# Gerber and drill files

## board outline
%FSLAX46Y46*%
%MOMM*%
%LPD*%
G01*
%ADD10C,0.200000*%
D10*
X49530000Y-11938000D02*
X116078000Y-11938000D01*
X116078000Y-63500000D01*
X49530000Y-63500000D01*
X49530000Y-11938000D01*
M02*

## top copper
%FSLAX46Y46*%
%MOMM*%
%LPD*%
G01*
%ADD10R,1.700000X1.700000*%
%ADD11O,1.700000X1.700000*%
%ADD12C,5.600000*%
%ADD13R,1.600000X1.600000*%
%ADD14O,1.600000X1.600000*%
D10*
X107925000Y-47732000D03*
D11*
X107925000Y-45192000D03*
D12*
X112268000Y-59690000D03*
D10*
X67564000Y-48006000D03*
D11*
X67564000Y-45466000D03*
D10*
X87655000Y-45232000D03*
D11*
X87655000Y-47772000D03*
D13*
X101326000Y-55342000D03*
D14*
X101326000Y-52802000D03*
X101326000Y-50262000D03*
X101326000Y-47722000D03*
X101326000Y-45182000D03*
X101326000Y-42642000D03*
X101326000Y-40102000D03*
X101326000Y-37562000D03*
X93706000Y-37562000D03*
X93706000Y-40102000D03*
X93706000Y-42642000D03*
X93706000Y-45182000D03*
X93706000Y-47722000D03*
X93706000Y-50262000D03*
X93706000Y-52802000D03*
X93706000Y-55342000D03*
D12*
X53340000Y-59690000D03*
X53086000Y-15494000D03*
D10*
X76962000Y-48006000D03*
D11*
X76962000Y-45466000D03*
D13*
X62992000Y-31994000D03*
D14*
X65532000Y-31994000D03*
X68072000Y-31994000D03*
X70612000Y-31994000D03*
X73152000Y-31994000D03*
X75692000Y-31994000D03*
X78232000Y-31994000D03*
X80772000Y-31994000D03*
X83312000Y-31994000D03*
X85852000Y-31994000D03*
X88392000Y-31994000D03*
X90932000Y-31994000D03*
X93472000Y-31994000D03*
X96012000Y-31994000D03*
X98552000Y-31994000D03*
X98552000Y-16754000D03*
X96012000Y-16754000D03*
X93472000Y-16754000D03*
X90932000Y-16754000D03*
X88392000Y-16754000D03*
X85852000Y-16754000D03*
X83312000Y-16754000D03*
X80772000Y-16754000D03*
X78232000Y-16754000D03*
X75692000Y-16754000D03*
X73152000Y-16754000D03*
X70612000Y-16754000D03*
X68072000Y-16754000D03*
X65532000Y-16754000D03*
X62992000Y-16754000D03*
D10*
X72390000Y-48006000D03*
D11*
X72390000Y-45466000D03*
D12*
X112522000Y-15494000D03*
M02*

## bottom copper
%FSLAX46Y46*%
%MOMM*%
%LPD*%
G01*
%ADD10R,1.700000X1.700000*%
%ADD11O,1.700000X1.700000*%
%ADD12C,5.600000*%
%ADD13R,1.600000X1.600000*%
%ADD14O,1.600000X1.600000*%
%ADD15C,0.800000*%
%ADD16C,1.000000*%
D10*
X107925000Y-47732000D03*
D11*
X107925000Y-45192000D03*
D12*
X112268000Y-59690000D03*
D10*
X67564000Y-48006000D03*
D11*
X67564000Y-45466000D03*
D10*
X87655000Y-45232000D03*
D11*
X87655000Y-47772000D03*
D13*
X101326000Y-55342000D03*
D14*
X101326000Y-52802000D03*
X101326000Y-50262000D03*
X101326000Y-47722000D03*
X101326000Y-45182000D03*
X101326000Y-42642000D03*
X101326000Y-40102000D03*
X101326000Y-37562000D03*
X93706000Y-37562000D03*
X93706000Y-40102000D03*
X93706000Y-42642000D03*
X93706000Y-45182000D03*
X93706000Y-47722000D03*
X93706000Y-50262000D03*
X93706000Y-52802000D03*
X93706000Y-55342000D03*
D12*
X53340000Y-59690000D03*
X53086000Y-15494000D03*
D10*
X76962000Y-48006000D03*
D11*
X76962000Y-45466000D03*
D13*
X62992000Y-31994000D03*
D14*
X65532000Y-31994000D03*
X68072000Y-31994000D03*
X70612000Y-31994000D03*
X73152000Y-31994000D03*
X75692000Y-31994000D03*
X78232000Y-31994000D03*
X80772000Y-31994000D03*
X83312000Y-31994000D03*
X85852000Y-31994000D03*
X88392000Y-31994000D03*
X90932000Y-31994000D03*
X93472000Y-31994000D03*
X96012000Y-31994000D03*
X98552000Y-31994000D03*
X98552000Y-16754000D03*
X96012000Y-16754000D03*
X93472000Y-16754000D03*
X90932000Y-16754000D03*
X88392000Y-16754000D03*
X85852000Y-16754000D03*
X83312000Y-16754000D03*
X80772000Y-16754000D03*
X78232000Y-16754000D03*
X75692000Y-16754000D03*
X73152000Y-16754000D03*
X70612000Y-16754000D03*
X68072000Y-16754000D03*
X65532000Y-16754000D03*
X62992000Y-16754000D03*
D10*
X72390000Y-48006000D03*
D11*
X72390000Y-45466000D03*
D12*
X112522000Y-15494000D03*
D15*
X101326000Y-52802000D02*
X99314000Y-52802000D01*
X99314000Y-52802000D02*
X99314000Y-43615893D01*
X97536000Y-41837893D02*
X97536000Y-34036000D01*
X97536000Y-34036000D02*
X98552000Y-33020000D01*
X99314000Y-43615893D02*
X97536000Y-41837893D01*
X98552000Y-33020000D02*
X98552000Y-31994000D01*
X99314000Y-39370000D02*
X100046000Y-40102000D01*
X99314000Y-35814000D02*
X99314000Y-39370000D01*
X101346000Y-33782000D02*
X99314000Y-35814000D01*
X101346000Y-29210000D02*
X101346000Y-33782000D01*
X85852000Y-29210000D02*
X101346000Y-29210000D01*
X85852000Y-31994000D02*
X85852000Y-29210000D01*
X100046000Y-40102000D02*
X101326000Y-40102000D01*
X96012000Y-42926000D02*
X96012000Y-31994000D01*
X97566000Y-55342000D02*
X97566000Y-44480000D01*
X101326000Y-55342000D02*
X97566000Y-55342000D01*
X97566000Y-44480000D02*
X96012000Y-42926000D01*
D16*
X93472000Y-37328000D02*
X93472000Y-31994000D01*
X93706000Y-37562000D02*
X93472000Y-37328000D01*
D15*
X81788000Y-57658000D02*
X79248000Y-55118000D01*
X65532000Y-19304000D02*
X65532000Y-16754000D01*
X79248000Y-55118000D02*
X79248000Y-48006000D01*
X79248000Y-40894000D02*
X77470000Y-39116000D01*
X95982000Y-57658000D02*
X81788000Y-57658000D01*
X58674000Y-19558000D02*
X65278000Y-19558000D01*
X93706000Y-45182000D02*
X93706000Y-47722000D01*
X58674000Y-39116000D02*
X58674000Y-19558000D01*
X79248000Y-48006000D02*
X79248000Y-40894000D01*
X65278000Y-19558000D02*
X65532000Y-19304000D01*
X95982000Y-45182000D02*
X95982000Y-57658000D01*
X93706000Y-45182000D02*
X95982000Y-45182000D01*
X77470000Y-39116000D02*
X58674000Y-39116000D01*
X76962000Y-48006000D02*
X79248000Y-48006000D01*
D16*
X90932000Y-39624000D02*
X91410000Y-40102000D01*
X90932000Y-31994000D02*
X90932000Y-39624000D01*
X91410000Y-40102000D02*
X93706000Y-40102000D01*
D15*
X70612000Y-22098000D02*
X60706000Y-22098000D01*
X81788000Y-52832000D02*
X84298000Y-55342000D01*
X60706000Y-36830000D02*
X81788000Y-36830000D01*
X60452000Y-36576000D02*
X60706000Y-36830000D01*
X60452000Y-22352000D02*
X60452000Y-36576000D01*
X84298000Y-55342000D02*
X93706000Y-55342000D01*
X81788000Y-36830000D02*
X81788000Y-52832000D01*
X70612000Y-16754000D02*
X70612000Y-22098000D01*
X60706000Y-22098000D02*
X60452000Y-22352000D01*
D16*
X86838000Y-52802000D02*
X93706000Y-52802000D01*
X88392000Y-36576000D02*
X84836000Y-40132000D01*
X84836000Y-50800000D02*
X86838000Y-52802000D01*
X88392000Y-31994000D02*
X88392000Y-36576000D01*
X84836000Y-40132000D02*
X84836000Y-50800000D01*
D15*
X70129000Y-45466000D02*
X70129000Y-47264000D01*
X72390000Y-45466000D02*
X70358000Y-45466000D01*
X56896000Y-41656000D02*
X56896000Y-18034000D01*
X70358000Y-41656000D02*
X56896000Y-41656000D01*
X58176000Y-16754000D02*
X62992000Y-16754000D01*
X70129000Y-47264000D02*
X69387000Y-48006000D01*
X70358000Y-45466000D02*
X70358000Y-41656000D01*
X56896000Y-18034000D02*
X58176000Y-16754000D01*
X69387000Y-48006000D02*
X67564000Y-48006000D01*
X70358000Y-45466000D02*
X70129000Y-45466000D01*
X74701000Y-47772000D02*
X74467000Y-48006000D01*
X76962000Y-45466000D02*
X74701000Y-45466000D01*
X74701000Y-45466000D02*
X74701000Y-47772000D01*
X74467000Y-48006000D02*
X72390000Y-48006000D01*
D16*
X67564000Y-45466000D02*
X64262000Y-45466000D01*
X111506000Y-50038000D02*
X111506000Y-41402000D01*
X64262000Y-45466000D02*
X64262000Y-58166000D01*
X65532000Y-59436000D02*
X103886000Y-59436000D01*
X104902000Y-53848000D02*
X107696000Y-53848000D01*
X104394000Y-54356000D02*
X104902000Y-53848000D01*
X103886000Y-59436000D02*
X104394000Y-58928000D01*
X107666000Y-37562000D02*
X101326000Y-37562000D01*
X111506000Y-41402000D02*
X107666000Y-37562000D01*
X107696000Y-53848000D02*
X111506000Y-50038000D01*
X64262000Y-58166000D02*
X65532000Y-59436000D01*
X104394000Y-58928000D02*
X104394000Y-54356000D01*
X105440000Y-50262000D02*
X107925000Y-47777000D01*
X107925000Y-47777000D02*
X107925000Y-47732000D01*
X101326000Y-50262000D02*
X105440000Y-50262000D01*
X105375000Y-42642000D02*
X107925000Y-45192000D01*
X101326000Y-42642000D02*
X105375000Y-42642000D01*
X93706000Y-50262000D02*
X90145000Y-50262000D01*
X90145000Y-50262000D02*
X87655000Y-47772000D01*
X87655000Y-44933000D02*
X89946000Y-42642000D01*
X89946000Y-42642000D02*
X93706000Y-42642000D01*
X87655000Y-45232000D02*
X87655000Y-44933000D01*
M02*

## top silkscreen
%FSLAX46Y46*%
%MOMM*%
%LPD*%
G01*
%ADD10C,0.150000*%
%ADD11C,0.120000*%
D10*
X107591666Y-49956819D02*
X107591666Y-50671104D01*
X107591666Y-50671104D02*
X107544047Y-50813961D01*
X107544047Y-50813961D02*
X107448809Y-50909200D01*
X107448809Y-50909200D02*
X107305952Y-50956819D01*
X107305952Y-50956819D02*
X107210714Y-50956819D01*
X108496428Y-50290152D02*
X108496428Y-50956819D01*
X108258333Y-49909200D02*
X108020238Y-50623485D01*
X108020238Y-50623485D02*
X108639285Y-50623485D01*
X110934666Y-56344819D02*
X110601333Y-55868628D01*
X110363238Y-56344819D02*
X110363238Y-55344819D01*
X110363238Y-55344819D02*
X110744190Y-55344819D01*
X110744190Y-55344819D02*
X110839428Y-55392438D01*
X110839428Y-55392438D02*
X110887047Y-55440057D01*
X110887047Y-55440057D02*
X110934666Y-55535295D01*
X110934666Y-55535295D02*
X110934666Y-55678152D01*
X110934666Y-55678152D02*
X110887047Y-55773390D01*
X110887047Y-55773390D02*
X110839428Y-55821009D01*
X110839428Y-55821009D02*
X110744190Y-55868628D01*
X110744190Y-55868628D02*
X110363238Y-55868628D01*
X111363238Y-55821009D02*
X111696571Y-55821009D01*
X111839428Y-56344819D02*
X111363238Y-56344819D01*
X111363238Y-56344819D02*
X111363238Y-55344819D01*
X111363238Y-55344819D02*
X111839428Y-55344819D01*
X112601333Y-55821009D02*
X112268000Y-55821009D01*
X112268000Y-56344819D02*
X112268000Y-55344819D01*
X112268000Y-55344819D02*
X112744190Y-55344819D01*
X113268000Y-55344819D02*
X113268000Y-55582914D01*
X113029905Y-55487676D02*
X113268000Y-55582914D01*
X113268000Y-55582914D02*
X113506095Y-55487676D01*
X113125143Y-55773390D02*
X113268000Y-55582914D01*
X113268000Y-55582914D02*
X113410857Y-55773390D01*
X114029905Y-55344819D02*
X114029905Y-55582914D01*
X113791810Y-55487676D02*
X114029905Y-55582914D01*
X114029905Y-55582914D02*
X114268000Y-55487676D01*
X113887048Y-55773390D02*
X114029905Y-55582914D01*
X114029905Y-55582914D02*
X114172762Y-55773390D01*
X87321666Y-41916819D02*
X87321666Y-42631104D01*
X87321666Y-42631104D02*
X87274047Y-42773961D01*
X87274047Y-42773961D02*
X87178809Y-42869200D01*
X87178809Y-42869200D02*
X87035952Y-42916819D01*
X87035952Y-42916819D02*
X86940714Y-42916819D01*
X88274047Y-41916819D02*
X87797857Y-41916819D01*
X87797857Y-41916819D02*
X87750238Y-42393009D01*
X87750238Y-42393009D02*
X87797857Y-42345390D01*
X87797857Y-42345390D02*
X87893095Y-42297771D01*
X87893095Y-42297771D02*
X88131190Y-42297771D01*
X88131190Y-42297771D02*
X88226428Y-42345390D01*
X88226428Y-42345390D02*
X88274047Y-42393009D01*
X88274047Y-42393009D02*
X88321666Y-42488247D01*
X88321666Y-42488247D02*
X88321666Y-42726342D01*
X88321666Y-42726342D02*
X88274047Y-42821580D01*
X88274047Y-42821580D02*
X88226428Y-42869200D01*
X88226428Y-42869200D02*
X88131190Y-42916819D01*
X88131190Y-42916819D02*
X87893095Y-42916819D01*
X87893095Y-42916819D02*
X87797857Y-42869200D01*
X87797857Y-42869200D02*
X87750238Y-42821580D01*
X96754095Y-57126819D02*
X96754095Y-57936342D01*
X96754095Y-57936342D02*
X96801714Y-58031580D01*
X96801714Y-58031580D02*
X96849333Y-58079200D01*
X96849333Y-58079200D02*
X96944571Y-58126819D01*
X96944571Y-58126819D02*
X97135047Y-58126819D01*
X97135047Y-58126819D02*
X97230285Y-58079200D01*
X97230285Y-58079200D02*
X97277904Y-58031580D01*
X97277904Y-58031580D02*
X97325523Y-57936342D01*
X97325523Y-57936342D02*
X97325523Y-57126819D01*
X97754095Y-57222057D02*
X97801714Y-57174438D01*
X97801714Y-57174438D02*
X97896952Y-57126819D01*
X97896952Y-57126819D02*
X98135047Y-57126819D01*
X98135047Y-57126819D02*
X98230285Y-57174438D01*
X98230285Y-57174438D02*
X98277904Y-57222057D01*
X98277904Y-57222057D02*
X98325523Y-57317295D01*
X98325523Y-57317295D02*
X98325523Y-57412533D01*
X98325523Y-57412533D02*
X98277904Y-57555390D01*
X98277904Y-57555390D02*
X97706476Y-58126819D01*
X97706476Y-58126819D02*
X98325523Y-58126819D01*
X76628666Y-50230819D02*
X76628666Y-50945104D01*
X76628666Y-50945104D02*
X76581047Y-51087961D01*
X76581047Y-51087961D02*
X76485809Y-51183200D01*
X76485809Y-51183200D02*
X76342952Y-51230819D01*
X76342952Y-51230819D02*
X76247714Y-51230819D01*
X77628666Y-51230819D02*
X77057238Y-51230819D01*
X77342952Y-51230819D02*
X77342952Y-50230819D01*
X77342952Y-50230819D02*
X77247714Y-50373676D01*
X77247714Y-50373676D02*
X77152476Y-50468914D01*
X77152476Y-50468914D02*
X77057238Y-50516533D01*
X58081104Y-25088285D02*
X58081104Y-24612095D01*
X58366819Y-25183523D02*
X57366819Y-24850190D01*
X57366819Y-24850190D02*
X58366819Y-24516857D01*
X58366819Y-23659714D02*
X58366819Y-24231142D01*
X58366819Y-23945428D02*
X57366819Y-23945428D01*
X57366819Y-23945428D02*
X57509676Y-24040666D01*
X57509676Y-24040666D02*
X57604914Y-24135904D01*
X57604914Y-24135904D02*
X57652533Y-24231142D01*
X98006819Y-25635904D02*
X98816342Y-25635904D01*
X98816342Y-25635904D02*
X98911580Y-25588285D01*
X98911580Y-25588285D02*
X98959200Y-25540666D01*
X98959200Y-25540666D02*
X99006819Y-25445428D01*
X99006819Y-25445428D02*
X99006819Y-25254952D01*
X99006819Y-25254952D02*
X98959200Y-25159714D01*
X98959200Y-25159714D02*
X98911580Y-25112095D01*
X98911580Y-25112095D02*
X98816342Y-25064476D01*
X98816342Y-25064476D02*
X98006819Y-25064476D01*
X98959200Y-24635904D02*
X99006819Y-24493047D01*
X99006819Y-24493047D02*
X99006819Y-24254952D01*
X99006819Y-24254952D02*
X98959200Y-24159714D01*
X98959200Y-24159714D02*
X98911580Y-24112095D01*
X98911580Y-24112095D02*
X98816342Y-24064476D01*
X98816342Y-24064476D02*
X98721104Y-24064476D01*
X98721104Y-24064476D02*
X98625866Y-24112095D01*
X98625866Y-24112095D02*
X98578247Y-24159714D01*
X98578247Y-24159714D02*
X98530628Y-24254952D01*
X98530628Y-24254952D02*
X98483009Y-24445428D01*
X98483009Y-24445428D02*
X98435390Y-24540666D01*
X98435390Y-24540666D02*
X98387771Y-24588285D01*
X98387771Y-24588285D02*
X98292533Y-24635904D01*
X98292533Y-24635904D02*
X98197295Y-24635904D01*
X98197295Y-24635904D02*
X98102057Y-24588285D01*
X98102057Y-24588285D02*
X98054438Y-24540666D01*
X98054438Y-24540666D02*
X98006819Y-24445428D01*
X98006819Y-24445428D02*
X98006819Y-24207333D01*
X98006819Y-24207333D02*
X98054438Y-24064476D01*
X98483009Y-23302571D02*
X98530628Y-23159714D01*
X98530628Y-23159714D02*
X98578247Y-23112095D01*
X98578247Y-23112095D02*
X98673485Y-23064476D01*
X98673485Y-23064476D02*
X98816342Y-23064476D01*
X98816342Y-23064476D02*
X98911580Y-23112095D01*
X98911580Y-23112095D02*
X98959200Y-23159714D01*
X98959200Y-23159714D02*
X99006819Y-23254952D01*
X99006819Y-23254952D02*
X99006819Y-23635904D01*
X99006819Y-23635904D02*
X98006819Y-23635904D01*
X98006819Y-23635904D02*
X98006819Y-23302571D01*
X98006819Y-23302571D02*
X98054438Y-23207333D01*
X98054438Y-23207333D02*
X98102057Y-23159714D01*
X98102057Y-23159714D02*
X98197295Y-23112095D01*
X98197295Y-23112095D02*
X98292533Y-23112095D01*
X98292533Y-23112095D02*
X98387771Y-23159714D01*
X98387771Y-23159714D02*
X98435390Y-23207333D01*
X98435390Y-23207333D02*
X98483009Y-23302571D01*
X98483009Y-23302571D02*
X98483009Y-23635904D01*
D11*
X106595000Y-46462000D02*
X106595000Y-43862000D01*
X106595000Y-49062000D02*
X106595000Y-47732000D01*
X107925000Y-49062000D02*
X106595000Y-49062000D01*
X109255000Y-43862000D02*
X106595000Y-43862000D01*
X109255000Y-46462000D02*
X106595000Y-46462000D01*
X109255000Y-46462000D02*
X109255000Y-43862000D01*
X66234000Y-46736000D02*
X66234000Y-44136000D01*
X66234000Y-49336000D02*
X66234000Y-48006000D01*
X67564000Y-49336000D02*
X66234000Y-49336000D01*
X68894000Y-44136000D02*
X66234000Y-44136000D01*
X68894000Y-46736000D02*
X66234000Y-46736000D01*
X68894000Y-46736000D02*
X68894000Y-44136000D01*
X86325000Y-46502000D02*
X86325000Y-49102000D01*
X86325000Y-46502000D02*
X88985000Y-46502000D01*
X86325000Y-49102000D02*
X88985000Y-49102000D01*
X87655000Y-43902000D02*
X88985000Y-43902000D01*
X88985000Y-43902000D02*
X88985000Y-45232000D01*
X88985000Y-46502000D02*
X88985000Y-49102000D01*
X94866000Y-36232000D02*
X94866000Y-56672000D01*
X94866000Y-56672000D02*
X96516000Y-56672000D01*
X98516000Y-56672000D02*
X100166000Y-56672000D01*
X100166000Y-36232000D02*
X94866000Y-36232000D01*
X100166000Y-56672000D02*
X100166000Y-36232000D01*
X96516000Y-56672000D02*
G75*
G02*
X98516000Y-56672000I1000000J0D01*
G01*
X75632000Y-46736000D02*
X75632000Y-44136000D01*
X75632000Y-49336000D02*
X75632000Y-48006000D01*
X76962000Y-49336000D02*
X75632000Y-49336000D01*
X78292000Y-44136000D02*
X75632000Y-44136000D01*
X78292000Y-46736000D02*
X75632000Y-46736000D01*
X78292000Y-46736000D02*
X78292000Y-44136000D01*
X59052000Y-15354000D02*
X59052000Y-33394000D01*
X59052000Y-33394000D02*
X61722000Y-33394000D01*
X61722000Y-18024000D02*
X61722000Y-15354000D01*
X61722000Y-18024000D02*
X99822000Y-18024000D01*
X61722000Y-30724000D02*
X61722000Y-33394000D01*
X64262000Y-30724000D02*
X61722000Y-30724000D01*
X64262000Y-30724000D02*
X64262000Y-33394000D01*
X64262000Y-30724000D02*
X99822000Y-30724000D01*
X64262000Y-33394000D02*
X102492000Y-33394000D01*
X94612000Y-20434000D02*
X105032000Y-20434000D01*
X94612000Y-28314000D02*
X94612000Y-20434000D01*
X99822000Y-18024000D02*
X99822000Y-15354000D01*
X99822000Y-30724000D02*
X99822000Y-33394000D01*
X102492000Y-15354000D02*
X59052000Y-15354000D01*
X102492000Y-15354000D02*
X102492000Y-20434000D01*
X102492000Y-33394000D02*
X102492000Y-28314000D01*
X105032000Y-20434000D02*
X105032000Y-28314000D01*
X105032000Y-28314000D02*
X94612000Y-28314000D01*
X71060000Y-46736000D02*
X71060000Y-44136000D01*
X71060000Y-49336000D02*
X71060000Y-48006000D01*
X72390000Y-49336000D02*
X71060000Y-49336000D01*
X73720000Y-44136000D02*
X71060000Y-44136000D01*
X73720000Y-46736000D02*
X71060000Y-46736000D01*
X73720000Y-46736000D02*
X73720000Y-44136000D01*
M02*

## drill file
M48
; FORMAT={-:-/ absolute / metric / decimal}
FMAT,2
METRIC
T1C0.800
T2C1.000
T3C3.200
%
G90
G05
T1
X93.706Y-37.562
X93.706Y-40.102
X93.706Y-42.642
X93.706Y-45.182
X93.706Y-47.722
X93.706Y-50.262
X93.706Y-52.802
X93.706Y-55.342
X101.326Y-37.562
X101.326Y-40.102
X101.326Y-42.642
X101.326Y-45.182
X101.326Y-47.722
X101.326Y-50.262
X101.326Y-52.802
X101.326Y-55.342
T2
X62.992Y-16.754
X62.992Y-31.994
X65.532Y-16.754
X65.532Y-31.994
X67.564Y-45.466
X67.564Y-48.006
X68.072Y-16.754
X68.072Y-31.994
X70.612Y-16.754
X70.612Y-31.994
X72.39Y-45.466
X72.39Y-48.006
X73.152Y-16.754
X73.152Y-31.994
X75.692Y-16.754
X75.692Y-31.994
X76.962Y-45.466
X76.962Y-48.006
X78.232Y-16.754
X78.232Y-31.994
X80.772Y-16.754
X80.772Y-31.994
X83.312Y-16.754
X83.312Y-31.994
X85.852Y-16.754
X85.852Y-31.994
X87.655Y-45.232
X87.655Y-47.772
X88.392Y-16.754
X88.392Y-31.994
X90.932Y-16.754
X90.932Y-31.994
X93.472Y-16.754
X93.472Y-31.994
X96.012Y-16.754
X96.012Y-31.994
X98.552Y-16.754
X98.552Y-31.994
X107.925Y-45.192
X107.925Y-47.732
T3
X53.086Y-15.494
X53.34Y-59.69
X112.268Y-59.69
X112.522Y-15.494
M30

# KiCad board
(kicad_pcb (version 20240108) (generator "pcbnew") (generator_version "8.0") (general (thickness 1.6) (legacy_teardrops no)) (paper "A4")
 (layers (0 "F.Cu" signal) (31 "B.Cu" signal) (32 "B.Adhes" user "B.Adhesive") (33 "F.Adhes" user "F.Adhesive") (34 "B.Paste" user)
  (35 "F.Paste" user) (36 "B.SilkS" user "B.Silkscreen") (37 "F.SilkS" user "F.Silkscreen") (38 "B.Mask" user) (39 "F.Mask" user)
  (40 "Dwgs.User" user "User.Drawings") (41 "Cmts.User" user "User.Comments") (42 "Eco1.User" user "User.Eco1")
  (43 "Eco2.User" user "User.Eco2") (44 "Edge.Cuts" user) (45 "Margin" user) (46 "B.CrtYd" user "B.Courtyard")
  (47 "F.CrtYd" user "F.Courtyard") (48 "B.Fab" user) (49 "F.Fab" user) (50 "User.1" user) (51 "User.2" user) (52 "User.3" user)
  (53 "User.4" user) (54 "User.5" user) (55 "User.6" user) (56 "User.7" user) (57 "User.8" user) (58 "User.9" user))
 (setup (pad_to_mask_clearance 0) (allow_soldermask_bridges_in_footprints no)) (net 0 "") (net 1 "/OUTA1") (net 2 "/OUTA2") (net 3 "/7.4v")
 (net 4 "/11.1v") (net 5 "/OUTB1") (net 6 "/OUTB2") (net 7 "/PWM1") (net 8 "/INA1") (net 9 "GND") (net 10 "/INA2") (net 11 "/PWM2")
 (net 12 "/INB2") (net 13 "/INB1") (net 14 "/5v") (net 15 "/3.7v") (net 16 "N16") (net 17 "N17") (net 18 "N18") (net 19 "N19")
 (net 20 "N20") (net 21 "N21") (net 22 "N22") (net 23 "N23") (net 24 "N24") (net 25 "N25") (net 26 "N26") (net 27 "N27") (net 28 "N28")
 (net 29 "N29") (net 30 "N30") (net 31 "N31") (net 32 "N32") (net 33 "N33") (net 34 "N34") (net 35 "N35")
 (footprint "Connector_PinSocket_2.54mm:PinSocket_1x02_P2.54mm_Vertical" (layer "F.Cu") (at 107.925 47.732 180)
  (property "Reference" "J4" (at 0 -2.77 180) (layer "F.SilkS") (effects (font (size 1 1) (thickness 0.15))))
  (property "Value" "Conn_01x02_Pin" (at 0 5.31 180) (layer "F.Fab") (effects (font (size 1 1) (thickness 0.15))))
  (fp_line (start 1.33 1.27) (end 1.33 3.87) (stroke (width 0.12) (type solid)) (layer "F.SilkS"))
  (fp_line (start 1.33 -1.33) (end 1.33 0) (stroke (width 0.12) (type solid)) (layer "F.SilkS"))
  (fp_line (start 0 -1.33) (end 1.33 -1.33) (stroke (width 0.12) (type solid)) (layer "F.SilkS"))
  (fp_line (start -1.33 3.87) (end 1.33 3.87) (stroke (width 0.12) (type solid)) (layer "F.SilkS"))
  (fp_line (start -1.33 1.27) (end 1.33 1.27) (stroke (width 0.12) (type solid)) (layer "F.SilkS"))
  (fp_line (start -1.33 1.27) (end -1.33 3.87) (stroke (width 0.12) (type solid)) (layer "F.SilkS"))
  (pad "1" thru_hole rect (at 0 0 180) (size 1.7 1.7) (drill 1) (layers "*.Cu" "*.Mask") (remove_unused_layers no) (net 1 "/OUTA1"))
  (pad "2" thru_hole oval (at 0 2.54 180) (size 1.7 1.7) (drill 1) (layers "*.Cu" "*.Mask") (remove_unused_layers no) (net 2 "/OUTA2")))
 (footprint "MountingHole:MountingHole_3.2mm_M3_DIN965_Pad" (layer "F.Cu") (at 112.268 59.69)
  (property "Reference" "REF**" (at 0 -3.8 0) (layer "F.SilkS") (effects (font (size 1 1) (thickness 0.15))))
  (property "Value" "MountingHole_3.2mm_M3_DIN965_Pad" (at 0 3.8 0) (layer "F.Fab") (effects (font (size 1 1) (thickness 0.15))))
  (pad "1" thru_hole circle (at 0 0) (size 5.6 5.6) (drill 3.2) (layers "*.Cu" "*.Mask") (remove_unused_layers no)))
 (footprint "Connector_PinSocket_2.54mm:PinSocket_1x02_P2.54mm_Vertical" (layer "F.Cu") (at 67.564 48.006 180)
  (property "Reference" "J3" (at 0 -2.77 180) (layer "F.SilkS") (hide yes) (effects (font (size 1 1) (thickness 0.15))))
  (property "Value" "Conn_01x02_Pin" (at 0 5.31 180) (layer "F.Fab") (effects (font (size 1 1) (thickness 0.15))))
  (fp_line (start 1.33 1.27) (end 1.33 3.87) (stroke (width 0.12) (type solid)) (layer "F.SilkS"))
  (fp_line (start 1.33 -1.33) (end 1.33 0) (stroke (width 0.12) (type solid)) (layer "F.SilkS"))
  (fp_line (start 0 -1.33) (end 1.33 -1.33) (stroke (width 0.12) (type solid)) (layer "F.SilkS"))
  (fp_line (start -1.33 3.87) (end 1.33 3.87) (stroke (width 0.12) (type solid)) (layer "F.SilkS"))
  (fp_line (start -1.33 1.27) (end 1.33 1.27) (stroke (width 0.12) (type solid)) (layer "F.SilkS"))
  (fp_line (start -1.33 1.27) (end -1.33 3.87) (stroke (width 0.12) (type solid)) (layer "F.SilkS"))
  (pad "1" thru_hole rect (at 0 0 180) (size 1.7 1.7) (drill 1) (layers "*.Cu" "*.Mask") (remove_unused_layers no) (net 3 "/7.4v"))
  (pad "2" thru_hole oval (at 0 2.54 180) (size 1.7 1.7) (drill 1) (layers "*.Cu" "*.Mask") (remove_unused_layers no) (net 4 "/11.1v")))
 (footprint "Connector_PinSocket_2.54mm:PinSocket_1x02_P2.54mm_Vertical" (layer "F.Cu") (at 87.655 45.232)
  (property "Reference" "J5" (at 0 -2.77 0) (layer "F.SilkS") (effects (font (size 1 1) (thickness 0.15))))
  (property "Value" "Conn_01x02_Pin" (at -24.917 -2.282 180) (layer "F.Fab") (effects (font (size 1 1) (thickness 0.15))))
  (fp_line (start -1.33 1.27) (end -1.33 3.87) (stroke (width 0.12) (type solid)) (layer "F.SilkS"))
  (fp_line (start -1.33 1.27) (end 1.33 1.27) (stroke (width 0.12) (type solid)) (layer "F.SilkS"))
  (fp_line (start -1.33 3.87) (end 1.33 3.87) (stroke (width 0.12) (type solid)) (layer "F.SilkS"))
  (fp_line (start 0 -1.33) (end 1.33 -1.33) (stroke (width 0.12) (type solid)) (layer "F.SilkS"))
  (fp_line (start 1.33 -1.33) (end 1.33 0) (stroke (width 0.12) (type solid)) (layer "F.SilkS"))
  (fp_line (start 1.33 1.27) (end 1.33 3.87) (stroke (width 0.12) (type solid)) (layer "F.SilkS"))
  (pad "1" thru_hole rect (at 0 0) (size 1.7 1.7) (drill 1) (layers "*.Cu" "*.Mask") (remove_unused_layers no) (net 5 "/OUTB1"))
  (pad "2" thru_hole oval (at 0 2.54) (size 1.7 1.7) (drill 1) (layers "*.Cu" "*.Mask") (remove_unused_layers no) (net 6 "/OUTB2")))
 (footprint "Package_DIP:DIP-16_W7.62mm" (layer "F.Cu") (at 101.326 55.342 180)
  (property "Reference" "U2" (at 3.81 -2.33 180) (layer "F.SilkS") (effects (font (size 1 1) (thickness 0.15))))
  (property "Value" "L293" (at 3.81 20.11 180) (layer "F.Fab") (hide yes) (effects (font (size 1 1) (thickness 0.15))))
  (fp_line (start 6.46 19.11) (end 6.46 -1.33) (stroke (width 0.12) (type solid)) (layer "F.SilkS"))
  (fp_line (start 6.46 -1.33) (end 4.81 -1.33) (stroke (width 0.12) (type solid)) (layer "F.SilkS"))
  (fp_line (start 2.81 -1.33) (end 1.16 -1.33) (stroke (width 0.12) (type solid)) (layer "F.SilkS"))
  (fp_line (start 1.16 19.11) (end 6.46 19.11) (stroke (width 0.12) (type solid)) (layer "F.SilkS"))
  (fp_line (start 1.16 -1.33) (end 1.16 19.11) (stroke (width 0.12) (type solid)) (layer "F.SilkS"))
  (fp_arc (start 4.81 -1.33) (mid 3.81 -0.33) (end 2.81 -1.33) (stroke (width 0.12) (type solid)) (layer "F.SilkS"))
  (pad "1" thru_hole rect (at 0 0 180) (size 1.6 1.6) (drill 0.8) (layers "*.Cu" "*.Mask") (remove_unused_layers no) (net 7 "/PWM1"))
  (pad "2" thru_hole oval (at 0 2.54 180) (size 1.6 1.6) (drill 0.8) (layers "*.Cu" "*.Mask") (remove_unused_layers no) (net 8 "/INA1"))
  (pad "3" thru_hole oval (at 0 5.08 180) (size 1.6 1.6) (drill 0.8) (layers "*.Cu" "*.Mask") (remove_unused_layers no) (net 1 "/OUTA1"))
  (pad "4" thru_hole oval (at 0 7.62 180) (size 1.6 1.6) (drill 0.8) (layers "*.Cu" "*.Mask") (remove_unused_layers no) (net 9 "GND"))
  (pad "5" thru_hole oval (at 0 10.16 180) (size 1.6 1.6) (drill 0.8) (layers "*.Cu" "*.Mask") (remove_unused_layers no) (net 9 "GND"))
  (pad "6" thru_hole oval (at 0 12.7 180) (size 1.6 1.6) (drill 0.8) (layers "*.Cu" "*.Mask") (remove_unused_layers no) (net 2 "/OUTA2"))
  (pad "7" thru_hole oval (at 0 15.24 180) (size 1.6 1.6) (drill 0.8) (layers "*.Cu" "*.Mask") (remove_unused_layers no) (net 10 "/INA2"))
  (pad "8" thru_hole oval (at 0 17.78 180) (size 1.6 1.6) (drill 0.8) (layers "*.Cu" "*.Mask") (remove_unused_layers no) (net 4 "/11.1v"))
  (pad "9" thru_hole oval (at 7.62 17.78 180) (size 1.6 1.6) (drill 0.8) (layers "*.Cu" "*.Mask") (remove_unused_layers no) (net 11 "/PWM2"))
  (pad "10" thru_hole oval (at 7.62 15.24 180) (size 1.6 1.6) (drill 0.8) (layers "*.Cu" "*.Mask") (remove_unused_layers no)
   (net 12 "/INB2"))
  (pad "11" thru_hole oval (at 7.62 12.7 180) (size 1.6 1.6) (drill 0.8) (layers "*.Cu" "*.Mask") (remove_unused_layers no) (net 5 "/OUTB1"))
  (pad "12" thru_hole oval (at 7.62 10.16 180) (size 1.6 1.6) (drill 0.8) (layers "*.Cu" "*.Mask") (remove_unused_layers no) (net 9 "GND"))
  (pad "13" thru_hole oval (at 7.62 7.62 180) (size 1.6 1.6) (drill 0.8) (layers "*.Cu" "*.Mask") (remove_unused_layers no) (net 9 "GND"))
  (pad "14" thru_hole oval (at 7.62 5.08 180) (size 1.6 1.6) (drill 0.8) (layers "*.Cu" "*.Mask") (remove_unused_layers no) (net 6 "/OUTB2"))
  (pad "15" thru_hole oval (at 7.62 2.54 180) (size 1.6 1.6) (drill 0.8) (layers "*.Cu" "*.Mask") (remove_unused_layers no) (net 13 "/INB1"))
  (pad "16" thru_hole oval (at 7.62 0 180) (size 1.6 1.6) (drill 0.8) (layers "*.Cu" "*.Mask") (remove_unused_layers no) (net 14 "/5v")))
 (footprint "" (layer "F.Cu") (at 53.34 59.69)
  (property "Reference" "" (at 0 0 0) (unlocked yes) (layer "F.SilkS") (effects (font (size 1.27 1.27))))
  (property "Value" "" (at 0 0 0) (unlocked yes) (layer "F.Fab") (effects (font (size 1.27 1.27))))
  (pad "1" thru_hole circle (at 0 0) (size 5.6 5.6) (drill 3.2) (layers "*.Cu" "*.Mask") (remove_unused_layers no)))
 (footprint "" (layer "F.Cu") (at 53.086 15.494)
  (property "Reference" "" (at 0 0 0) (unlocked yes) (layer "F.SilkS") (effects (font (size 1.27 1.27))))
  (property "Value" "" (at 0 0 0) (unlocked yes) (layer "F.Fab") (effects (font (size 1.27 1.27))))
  (pad "1" thru_hole circle (at 0 0) (size 5.6 5.6) (drill 3.2) (layers "*.Cu" "*.Mask") (remove_unused_layers no)))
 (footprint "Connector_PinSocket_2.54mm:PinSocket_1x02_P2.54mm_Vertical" (layer "F.Cu") (at 76.962 48.006 180)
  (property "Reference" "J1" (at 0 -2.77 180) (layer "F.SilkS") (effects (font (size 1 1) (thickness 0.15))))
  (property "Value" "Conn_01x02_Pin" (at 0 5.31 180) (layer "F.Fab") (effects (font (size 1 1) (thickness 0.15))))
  (fp_line (start 1.33 1.27) (end 1.33 3.87) (stroke (width 0.12) (type solid)) (layer "F.SilkS"))
  (fp_line (start 1.33 -1.33) (end 1.33 0) (stroke (width 0.12) (type solid)) (layer "F.SilkS"))
  (fp_line (start 0 -1.33) (end 1.33 -1.33) (stroke (width 0.12) (type solid)) (layer "F.SilkS"))
  (fp_line (start -1.33 3.87) (end 1.33 3.87) (stroke (width 0.12) (type solid)) (layer "F.SilkS"))
  (fp_line (start -1.33 1.27) (end 1.33 1.27) (stroke (width 0.12) (type solid)) (layer "F.SilkS"))
  (fp_line (start -1.33 1.27) (end -1.33 3.87) (stroke (width 0.12) (type solid)) (layer "F.SilkS"))
  (pad "1" thru_hole rect (at 0 0 180) (size 1.7 1.7) (drill 1) (layers "*.Cu" "*.Mask") (remove_unused_layers no) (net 9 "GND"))
  (pad "2" thru_hole oval (at 0 2.54 180) (size 1.7 1.7) (drill 1) (layers "*.Cu" "*.Mask") (remove_unused_layers no) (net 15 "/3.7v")))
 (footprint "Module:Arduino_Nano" (layer "F.Cu") (at 62.992 31.994 90)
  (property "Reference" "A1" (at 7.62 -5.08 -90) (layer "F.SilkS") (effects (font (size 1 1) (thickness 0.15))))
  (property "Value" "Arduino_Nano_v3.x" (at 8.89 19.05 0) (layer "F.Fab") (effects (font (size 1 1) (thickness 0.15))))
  (fp_line (start 16.64 -3.94) (end -1.4 -3.94) (stroke (width 0.12) (type solid)) (layer "F.SilkS"))
  (fp_line (start -1.4 -3.94) (end -1.4 -1.27) (stroke (width 0.12) (type solid)) (layer "F.SilkS"))
  (fp_line (start 13.97 -1.27) (end 16.64 -1.27) (stroke (width 0.12) (type solid)) (layer "F.SilkS"))
  (fp_line (start 13.97 -1.27) (end 13.97 36.83) (stroke (width 0.12) (type solid)) (layer "F.SilkS"))
  (fp_line (start 1.27 -1.27) (end -1.4 -1.27) (stroke (width 0.12) (type solid)) (layer "F.SilkS"))
  (fp_line (start 1.27 1.27) (end 1.27 -1.27) (stroke (width 0.12) (type solid)) (layer "F.SilkS"))
  (fp_line (start 1.27 1.27) (end -1.4 1.27) (stroke (width 0.12) (type solid)) (layer "F.SilkS"))
  (fp_line (start 1.27 1.27) (end 1.27 36.83) (stroke (width 0.12) (type solid)) (layer "F.SilkS"))
  (fp_line (start -1.4 1.27) (end -1.4 39.5) (stroke (width 0.12) (type solid)) (layer "F.SilkS"))
  (fp_line (start 11.56 31.62) (end 11.56 42.04) (stroke (width 0.12) (type solid)) (layer "F.SilkS"))
  (fp_line (start 3.68 31.62) (end 11.56 31.62) (stroke (width 0.12) (type solid)) (layer "F.SilkS"))
  (fp_line (start 13.97 36.83) (end 16.64 36.83) (stroke (width 0.12) (type solid)) (layer "F.SilkS"))
  (fp_line (start 1.27 36.83) (end -1.4 36.83) (stroke (width 0.12) (type solid)) (layer "F.SilkS"))
  (fp_line (start 16.64 39.5) (end 16.64 -3.94) (stroke (width 0.12) (type solid)) (layer "F.SilkS"))
  (fp_line (start 16.64 39.5) (end 11.56 39.5) (stroke (width 0.12) (type solid)) (layer "F.SilkS"))
  (fp_line (start -1.4 39.5) (end 3.68 39.5) (stroke (width 0.12) (type solid)) (layer "F.SilkS"))
  (fp_line (start 11.56 42.04) (end 3.68 42.04) (stroke (width 0.12) (type solid)) (layer "F.SilkS"))
  (fp_line (start 3.68 42.04) (end 3.68 31.62) (stroke (width 0.12) (type solid)) (layer "F.SilkS"))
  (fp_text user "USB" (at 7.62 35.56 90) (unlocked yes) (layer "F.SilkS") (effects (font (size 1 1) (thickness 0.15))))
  (pad "1" thru_hole rect (at 0 0 90) (size 1.6 1.6) (drill 1) (layers "*.Cu" "*.Mask") (remove_unused_layers no) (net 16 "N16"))
  (pad "2" thru_hole oval (at 0 2.54 90) (size 1.6 1.6) (drill 1) (layers "*.Cu" "*.Mask") (remove_unused_layers no) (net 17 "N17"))
  (pad "3" thru_hole oval (at 0 5.08 90) (size 1.6 1.6) (drill 1) (layers "*.Cu" "*.Mask") (remove_unused_layers no) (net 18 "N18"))
  (pad "4" thru_hole oval (at 0 7.62 90) (size 1.6 1.6) (drill 1) (layers "*.Cu" "*.Mask") (remove_unused_layers no) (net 9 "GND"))
  (pad "5" thru_hole oval (at 0 10.16 90) (size 1.6 1.6) (drill 1) (layers "*.Cu" "*.Mask") (remove_unused_layers no) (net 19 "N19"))
  (pad "6" thru_hole oval (at 0 12.7 90) (size 1.6 1.6) (drill 1) (layers "*.Cu" "*.Mask") (remove_unused_layers no) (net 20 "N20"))
  (pad "7" thru_hole oval (at 0 15.24 90) (size 1.6 1.6) (drill 1) (layers "*.Cu" "*.Mask") (remove_unused_layers no) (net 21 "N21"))
  (pad "8" thru_hole oval (at 0 17.78 90) (size 1.6 1.6) (drill 1) (layers "*.Cu" "*.Mask") (remove_unused_layers no) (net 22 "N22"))
  (pad "9" thru_hole oval (at 0 20.32 90) (size 1.6 1.6) (drill 1) (layers "*.Cu" "*.Mask") (remove_unused_layers no) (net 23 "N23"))
  (pad "10" thru_hole oval (at 0 22.86 90) (size 1.6 1.6) (drill 1) (layers "*.Cu" "*.Mask") (remove_unused_layers no) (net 10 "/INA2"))
  (pad "11" thru_hole oval (at 0 25.4 90) (size 1.6 1.6) (drill 1) (layers "*.Cu" "*.Mask") (remove_unused_layers no) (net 13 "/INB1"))
  (pad "12" thru_hole oval (at 0 27.94 90) (size 1.6 1.6) (drill 1) (layers "*.Cu" "*.Mask") (remove_unused_layers no) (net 12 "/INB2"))
  (pad "13" thru_hole oval (at 0 30.48 90) (size 1.6 1.6) (drill 1) (layers "*.Cu" "*.Mask") (remove_unused_layers no) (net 11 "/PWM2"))
  (pad "14" thru_hole oval (at 0 33.02 90) (size 1.6 1.6) (drill 1) (layers "*.Cu" "*.Mask") (remove_unused_layers no) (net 7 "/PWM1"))
  (pad "15" thru_hole oval (at 0 35.56 90) (size 1.6 1.6) (drill 1) (layers "*.Cu" "*.Mask") (remove_unused_layers no) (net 8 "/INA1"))
  (pad "16" thru_hole oval (at 15.24 35.56 90) (size 1.6 1.6) (drill 1) (layers "*.Cu" "*.Mask") (remove_unused_layers no) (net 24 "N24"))
  (pad "17" thru_hole oval (at 15.24 33.02 90) (size 1.6 1.6) (drill 1) (layers "*.Cu" "*.Mask") (remove_unused_layers no) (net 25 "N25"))
  (pad "18" thru_hole oval (at 15.24 30.48 90) (size 1.6 1.6) (drill 1) (layers "*.Cu" "*.Mask") (remove_unused_layers no) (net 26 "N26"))
  (pad "19" thru_hole oval (at 15.24 27.94 90) (size 1.6 1.6) (drill 1) (layers "*.Cu" "*.Mask") (remove_unused_layers no) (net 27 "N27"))
  (pad "20" thru_hole oval (at 15.24 25.4 90) (size 1.6 1.6) (drill 1) (layers "*.Cu" "*.Mask") (remove_unused_layers no) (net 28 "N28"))
  (pad "21" thru_hole oval (at 15.24 22.86 90) (size 1.6 1.6) (drill 1) (layers "*.Cu" "*.Mask") (remove_unused_layers no) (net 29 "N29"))
  (pad "22" thru_hole oval (at 15.24 20.32 90) (size 1.6 1.6) (drill 1) (layers "*.Cu" "*.Mask") (remove_unused_layers no) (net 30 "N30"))
  (pad "23" thru_hole oval (at 15.24 17.78 90) (size 1.6 1.6) (drill 1) (layers "*.Cu" "*.Mask") (remove_unused_layers no) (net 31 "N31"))
  (pad "24" thru_hole oval (at 15.24 15.24 90) (size 1.6 1.6) (drill 1) (layers "*.Cu" "*.Mask") (remove_unused_layers no) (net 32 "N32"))
  (pad "25" thru_hole oval (at 15.24 12.7 90) (size 1.6 1.6) (drill 1) (layers "*.Cu" "*.Mask") (remove_unused_layers no) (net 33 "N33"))
  (pad "26" thru_hole oval (at 15.24 10.16 90) (size 1.6 1.6) (drill 1) (layers "*.Cu" "*.Mask") (remove_unused_layers no) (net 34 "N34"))
  (pad "27" thru_hole oval (at 15.24 7.62 90) (size 1.6 1.6) (drill 1) (layers "*.Cu" "*.Mask") (remove_unused_layers no) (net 14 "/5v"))
  (pad "28" thru_hole oval (at 15.24 5.08 90) (size 1.6 1.6) (drill 1) (layers "*.Cu" "*.Mask") (remove_unused_layers no) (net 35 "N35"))
  (pad "29" thru_hole oval (at 15.24 2.54 90) (size 1.6 1.6) (drill 1) (layers "*.Cu" "*.Mask") (remove_unused_layers no) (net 9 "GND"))
  (pad "30" thru_hole oval (at 15.24 0 90) (size 1.6 1.6) (drill 1) (layers "*.Cu" "*.Mask") (remove_unused_layers no) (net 3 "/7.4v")))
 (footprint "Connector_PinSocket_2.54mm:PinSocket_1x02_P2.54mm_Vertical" (layer "F.Cu") (at 72.39 48.006 180)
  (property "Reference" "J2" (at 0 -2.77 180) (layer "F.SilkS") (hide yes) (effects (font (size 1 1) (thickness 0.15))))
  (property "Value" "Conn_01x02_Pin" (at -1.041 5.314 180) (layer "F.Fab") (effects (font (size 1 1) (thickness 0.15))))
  (fp_line (start 1.33 1.27) (end 1.33 3.87) (stroke (width 0.12) (type solid)) (layer "F.SilkS"))
  (fp_line (start 1.33 -1.33) (end 1.33 0) (stroke (width 0.12) (type solid)) (layer "F.SilkS"))
  (fp_line (start 0 -1.33) (end 1.33 -1.33) (stroke (width 0.12) (type solid)) (layer "F.SilkS"))
  (fp_line (start -1.33 3.87) (end 1.33 3.87) (stroke (width 0.12) (type solid)) (layer "F.SilkS"))
  (fp_line (start -1.33 1.27) (end 1.33 1.27) (stroke (width 0.12) (type solid)) (layer "F.SilkS"))
  (fp_line (start -1.33 1.27) (end -1.33 3.87) (stroke (width 0.12) (type solid)) (layer "F.SilkS"))
  (pad "1" thru_hole rect (at 0 0 180) (size 1.7 1.7) (drill 1) (layers "*.Cu" "*.Mask") (remove_unused_layers no) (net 15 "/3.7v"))
  (pad "2" thru_hole oval (at 0 2.54 180) (size 1.7 1.7) (drill 1) (layers "*.Cu" "*.Mask") (remove_unused_layers no) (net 3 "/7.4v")))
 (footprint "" (layer "F.Cu") (at 112.522 15.494)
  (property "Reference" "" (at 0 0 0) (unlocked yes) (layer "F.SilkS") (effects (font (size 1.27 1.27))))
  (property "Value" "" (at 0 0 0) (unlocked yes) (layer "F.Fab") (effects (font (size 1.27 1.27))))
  (pad "1" thru_hole circle (at 0 0) (size 5.6 5.6) (drill 3.2) (layers "*.Cu" "*.Mask") (remove_unused_layers no)))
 (gr_rect (start 49.53 11.938) (end 116.078 63.5) (stroke (width 0.2) (type default)) (fill none) (layer "Edge.Cuts"))
 (segment (start 101.326 52.802) (end 99.314 52.802) (width 0.8) (layer "B.Cu") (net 8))
 (segment (start 99.314 52.802) (end 99.314 43.615893) (width 0.8) (layer "B.Cu") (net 8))
 (segment (start 97.536 41.837893) (end 97.536 34.036) (width 0.8) (layer "B.Cu") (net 8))
 (segment (start 97.536 34.036) (end 98.552 33.02) (width 0.8) (layer "B.Cu") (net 8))
 (segment (start 99.314 43.615893) (end 97.536 41.837893) (width 0.8) (layer "B.Cu") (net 8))
 (segment (start 98.552 33.02) (end 98.552 31.994) (width 0.8) (layer "B.Cu") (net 8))
 (segment (start 99.314 39.37) (end 100.046 40.102) (width 0.8) (layer "B.Cu") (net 10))
 (segment (start 99.314 35.814) (end 99.314 39.37) (width 0.8) (layer "B.Cu") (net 10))
 (segment (start 101.346 33.782) (end 99.314 35.814) (width 0.8) (layer "B.Cu") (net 10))
 (segment (start 101.346 29.21) (end 101.346 33.782) (width 0.8) (layer "B.Cu") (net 10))
 (segment (start 85.852 29.21) (end 101.346 29.21) (width 0.8) (layer "B.Cu") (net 10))
 (segment (start 85.852 31.994) (end 85.852 29.21) (width 0.8) (layer "B.Cu") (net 10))
 (segment (start 100.046 40.102) (end 101.326 40.102) (width 0.8) (layer "B.Cu") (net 10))
 (segment (start 96.012 42.926) (end 96.012 31.994) (width 0.8) (layer "B.Cu") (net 7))
 (segment (start 97.566 55.342) (end 97.566 44.48) (width 0.8) (layer "B.Cu") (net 7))
 (segment (start 101.326 55.342) (end 97.566 55.342) (width 0.8) (layer "B.Cu") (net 7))
 (segment (start 97.566 44.48) (end 96.012 42.926) (width 0.8) (layer "B.Cu") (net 7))
 (segment (start 93.472 37.328) (end 93.472 31.994) (width 1) (layer "B.Cu") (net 11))
 (segment (start 93.706 37.562) (end 93.472 37.328) (width 1) (layer "B.Cu") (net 11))
 (segment (start 81.788 57.658) (end 79.248 55.118) (width 0.8) (layer "B.Cu") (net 9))
 (segment (start 65.532 19.304) (end 65.532 16.754) (width 0.8) (layer "B.Cu") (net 9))
 (segment (start 79.248 55.118) (end 79.248 48.006) (width 0.8) (layer "B.Cu") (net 9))
 (segment (start 79.248 40.894) (end 77.47 39.116) (width 0.8) (layer "B.Cu") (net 9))
 (segment (start 95.982 57.658) (end 81.788 57.658) (width 0.8) (layer "B.Cu") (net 9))
 (segment (start 58.674 19.558) (end 65.278 19.558) (width 0.8) (layer "B.Cu") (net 9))
 (segment (start 93.706 45.182) (end 93.706 47.722) (width 0.8) (layer "B.Cu") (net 9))
 (segment (start 58.674 39.116) (end 58.674 19.558) (width 0.8) (layer "B.Cu") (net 9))
 (segment (start 79.248 48.006) (end 79.248 40.894) (width 0.8) (layer "B.Cu") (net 9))
 (segment (start 65.278 19.558) (end 65.532 19.304) (width 0.8) (layer "B.Cu") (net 9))
 (segment (start 95.982 45.182) (end 95.982 57.658) (width 0.8) (layer "B.Cu") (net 9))
 (segment (start 93.706 45.182) (end 95.982 45.182) (width 0.8) (layer "B.Cu") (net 9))
 (segment (start 77.47 39.116) (end 58.674 39.116) (width 0.8) (layer "B.Cu") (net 9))
 (segment (start 76.962 48.006) (end 79.248 48.006) (width 0.8) (layer "B.Cu") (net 9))
 (segment (start 90.932 39.624) (end 91.41 40.102) (width 1) (layer "B.Cu") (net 12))
 (segment (start 90.932 31.994) (end 90.932 39.624) (width 1) (layer "B.Cu") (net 12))
 (segment (start 91.41 40.102) (end 93.706 40.102) (width 1) (layer "B.Cu") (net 12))
 (segment (start 70.612 22.098) (end 60.706 22.098) (width 0.8) (layer "B.Cu") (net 14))
 (segment (start 81.788 52.832) (end 84.298 55.342) (width 0.8) (layer "B.Cu") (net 14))
 (segment (start 60.706 36.83) (end 81.788 36.83) (width 0.8) (layer "B.Cu") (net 14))
 (segment (start 60.452 36.576) (end 60.706 36.83) (width 0.8) (layer "B.Cu") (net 14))
 (segment (start 60.452 22.352) (end 60.452 36.576) (width 0.8) (layer "B.Cu") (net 14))
 (segment (start 84.298 55.342) (end 93.706 55.342) (width 0.8) (layer "B.Cu") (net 14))
 (segment (start 81.788 36.83) (end 81.788 52.832) (width 0.8) (layer "B.Cu") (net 14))
 (segment (start 70.612 16.754) (end 70.612 22.098) (width 0.8) (layer "B.Cu") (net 14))
 (segment (start 60.706 22.098) (end 60.452 22.352) (width 0.8) (layer "B.Cu") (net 14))
 (segment (start 86.838 52.802) (end 93.706 52.802) (width 1) (layer "B.Cu") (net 13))
 (segment (start 88.392 36.576) (end 84.836 40.132) (width 1) (layer "B.Cu") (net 13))
 (segment (start 84.836 50.8) (end 86.838 52.802) (width 1) (layer "B.Cu") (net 13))
 (segment (start 88.392 31.994) (end 88.392 36.576) (width 1) (layer "B.Cu") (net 13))
 (segment (start 84.836 40.132) (end 84.836 50.8) (width 1) (layer "B.Cu") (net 13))
 (segment (start 70.129 45.466) (end 70.129 47.264) (width 0.8) (layer "B.Cu") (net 3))
 (segment (start 72.39 45.466) (end 70.358 45.466) (width 0.8) (layer "B.Cu") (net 3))
 (segment (start 56.896 41.656) (end 56.896 18.034) (width 0.8) (layer "B.Cu") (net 3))
 (segment (start 70.358 41.656) (end 56.896 41.656) (width 0.8) (layer "B.Cu") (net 3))
 (segment (start 58.176 16.754) (end 62.992 16.754) (width 0.8) (layer "B.Cu") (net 3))
 (segment (start 70.129 47.264) (end 69.387 48.006) (width 0.8) (layer "B.Cu") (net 3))
 (segment (start 70.358 45.466) (end 70.358 41.656) (width 0.8) (layer "B.Cu") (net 3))
 (segment (start 56.896 18.034) (end 58.176 16.754) (width 0.8) (layer "B.Cu") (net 3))
 (segment (start 69.387 48.006) (end 67.564 48.006) (width 0.8) (layer "B.Cu") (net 3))
 (segment (start 70.358 45.466) (end 70.129 45.466) (width 0.8) (layer "B.Cu") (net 3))
 (segment (start 74.701 47.772) (end 74.467 48.006) (width 0.8) (layer "B.Cu") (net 15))
 (segment (start 76.962 45.466) (end 74.701 45.466) (width 0.8) (layer "B.Cu") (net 15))
 (segment (start 74.701 45.466) (end 74.701 47.772) (width 0.8) (layer "B.Cu") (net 15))
 (segment (start 74.467 48.006) (end 72.39 48.006) (width 0.8) (layer "B.Cu") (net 15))
 (segment (start 67.564 45.466) (end 64.262 45.466) (width 1) (layer "B.Cu") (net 4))
 (segment (start 111.506 50.038) (end 111.506 41.402) (width 1) (layer "B.Cu") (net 4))
 (segment (start 64.262 45.466) (end 64.262 58.166) (width 1) (layer "B.Cu") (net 4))
 (segment (start 65.532 59.436) (end 103.886 59.436) (width 1) (layer "B.Cu") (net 4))
 (segment (start 104.902 53.848) (end 107.696 53.848) (width 1) (layer "B.Cu") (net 4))
 (segment (start 104.394 54.356) (end 104.902 53.848) (width 1) (layer "B.Cu") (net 4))
 (segment (start 103.886 59.436) (end 104.394 58.928) (width 1) (layer "B.Cu") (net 4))
 (segment (start 107.666 37.562) (end 101.326 37.562) (width 1) (layer "B.Cu") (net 4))
 (segment (start 111.506 41.402) (end 107.666 37.562) (width 1) (layer "B.Cu") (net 4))
 (segment (start 107.696 53.848) (end 111.506 50.038) (width 1) (layer "B.Cu") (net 4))
 (segment (start 64.262 58.166) (end 65.532 59.436) (width 1) (layer "B.Cu") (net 4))
 (segment (start 104.394 58.928) (end 104.394 54.356) (width 1) (layer "B.Cu") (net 4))
 (segment (start 105.44 50.262) (end 107.925 47.777) (width 1) (layer "B.Cu") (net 1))
 (segment (start 107.925 47.777) (end 107.925 47.732) (width 1) (layer "B.Cu") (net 1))
 (segment (start 101.326 50.262) (end 105.44 50.262) (width 1) (layer "B.Cu") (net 1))
 (segment (start 105.375 42.642) (end 107.925 45.192) (width 1) (layer "B.Cu") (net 2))
 (segment (start 101.326 42.642) (end 105.375 42.642) (width 1) (layer "B.Cu") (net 2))
 (segment (start 93.706 50.262) (end 90.145 50.262) (width 1) (layer "B.Cu") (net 6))
 (segment (start 90.145 50.262) (end 87.655 47.772) (width 1) (layer "B.Cu") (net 6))
 (segment (start 87.655 44.933) (end 89.946 42.642) (width 1) (layer "B.Cu") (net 5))
 (segment (start 89.946 42.642) (end 93.706 42.642) (width 1) (layer "B.Cu") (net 5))
 (segment (start 87.655 45.232) (end 87.655 44.933) (width 1) (layer "B.Cu") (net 5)))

